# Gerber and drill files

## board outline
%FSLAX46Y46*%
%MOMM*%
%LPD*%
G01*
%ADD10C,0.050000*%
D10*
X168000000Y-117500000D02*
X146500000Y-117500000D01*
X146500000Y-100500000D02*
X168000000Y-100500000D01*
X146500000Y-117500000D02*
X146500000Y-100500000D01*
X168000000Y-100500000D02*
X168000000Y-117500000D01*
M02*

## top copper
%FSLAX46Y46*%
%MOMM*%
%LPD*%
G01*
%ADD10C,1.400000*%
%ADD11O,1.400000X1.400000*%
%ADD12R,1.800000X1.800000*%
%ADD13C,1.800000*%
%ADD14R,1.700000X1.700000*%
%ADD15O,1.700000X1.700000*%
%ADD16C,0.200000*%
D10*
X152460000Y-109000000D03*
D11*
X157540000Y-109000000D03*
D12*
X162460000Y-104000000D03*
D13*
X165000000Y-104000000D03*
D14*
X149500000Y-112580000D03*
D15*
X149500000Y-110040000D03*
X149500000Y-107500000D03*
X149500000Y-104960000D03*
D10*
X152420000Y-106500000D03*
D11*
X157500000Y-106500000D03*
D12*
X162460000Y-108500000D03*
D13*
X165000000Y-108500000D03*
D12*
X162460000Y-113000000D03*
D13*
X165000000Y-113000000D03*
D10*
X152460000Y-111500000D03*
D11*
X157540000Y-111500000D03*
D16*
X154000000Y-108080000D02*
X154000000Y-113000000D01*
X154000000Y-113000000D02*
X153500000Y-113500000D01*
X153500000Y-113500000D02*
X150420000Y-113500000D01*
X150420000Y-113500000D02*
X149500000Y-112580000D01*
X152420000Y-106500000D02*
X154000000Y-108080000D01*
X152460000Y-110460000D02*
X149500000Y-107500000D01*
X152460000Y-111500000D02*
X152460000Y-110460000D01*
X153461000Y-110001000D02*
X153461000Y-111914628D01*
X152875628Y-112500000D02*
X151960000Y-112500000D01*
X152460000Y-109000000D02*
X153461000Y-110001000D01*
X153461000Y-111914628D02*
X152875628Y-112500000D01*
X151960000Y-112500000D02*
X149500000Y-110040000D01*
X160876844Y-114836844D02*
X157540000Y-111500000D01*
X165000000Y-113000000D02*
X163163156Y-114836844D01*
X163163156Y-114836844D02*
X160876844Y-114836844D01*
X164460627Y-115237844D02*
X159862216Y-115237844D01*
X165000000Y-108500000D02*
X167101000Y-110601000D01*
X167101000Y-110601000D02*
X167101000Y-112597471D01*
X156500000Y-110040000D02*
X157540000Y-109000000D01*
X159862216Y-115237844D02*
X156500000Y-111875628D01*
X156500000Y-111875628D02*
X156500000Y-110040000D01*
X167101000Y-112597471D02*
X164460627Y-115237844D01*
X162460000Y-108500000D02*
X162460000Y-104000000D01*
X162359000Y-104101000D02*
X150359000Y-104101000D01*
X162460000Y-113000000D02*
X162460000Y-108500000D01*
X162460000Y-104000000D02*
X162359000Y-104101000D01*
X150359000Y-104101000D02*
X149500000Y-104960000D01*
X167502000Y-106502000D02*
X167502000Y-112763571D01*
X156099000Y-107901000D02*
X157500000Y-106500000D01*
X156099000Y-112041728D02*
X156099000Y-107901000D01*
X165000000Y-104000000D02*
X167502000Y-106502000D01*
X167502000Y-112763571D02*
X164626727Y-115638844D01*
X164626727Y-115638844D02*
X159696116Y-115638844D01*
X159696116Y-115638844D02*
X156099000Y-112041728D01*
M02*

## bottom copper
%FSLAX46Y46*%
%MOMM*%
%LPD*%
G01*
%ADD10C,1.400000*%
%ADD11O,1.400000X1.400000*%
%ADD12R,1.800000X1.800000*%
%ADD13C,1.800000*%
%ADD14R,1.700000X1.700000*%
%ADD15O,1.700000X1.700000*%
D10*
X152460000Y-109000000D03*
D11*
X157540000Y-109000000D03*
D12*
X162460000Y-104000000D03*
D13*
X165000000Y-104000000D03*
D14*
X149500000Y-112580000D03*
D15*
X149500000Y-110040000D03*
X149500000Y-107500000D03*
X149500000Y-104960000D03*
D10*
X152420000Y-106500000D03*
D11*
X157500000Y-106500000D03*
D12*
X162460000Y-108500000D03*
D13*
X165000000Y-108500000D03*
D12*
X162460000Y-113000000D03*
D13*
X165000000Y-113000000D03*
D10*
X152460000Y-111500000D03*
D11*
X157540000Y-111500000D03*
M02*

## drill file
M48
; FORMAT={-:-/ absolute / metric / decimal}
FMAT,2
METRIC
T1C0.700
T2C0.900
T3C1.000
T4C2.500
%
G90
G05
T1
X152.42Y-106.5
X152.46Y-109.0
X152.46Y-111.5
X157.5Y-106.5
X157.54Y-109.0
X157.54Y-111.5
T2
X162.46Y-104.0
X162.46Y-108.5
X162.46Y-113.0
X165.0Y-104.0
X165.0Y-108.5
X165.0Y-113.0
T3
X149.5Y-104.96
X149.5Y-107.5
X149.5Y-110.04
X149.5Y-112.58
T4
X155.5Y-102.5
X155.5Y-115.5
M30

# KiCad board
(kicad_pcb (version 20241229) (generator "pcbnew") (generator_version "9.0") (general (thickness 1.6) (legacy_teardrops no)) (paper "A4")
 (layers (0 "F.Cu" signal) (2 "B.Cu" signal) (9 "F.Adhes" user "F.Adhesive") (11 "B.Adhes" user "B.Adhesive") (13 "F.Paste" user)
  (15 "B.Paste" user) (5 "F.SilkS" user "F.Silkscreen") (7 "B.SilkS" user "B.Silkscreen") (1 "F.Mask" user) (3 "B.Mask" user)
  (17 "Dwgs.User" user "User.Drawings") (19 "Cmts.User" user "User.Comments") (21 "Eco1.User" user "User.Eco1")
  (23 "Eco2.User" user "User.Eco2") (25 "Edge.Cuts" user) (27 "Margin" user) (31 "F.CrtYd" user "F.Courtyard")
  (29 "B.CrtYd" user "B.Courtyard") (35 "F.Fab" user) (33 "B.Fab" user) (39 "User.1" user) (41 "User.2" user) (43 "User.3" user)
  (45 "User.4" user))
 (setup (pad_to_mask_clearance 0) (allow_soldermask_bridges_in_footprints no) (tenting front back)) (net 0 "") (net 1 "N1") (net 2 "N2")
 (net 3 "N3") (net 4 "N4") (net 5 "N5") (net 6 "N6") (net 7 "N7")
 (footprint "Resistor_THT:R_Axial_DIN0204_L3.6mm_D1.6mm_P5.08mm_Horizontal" (layer "F.Cu") (at 152.46 109)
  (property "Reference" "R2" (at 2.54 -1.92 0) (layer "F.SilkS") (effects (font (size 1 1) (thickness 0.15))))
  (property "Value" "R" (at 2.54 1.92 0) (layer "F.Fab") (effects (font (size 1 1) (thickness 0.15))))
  (pad "1" thru_hole circle (at 0 0) (size 1.4 1.4) (drill 0.7) (layers "*.Cu" "*.Mask") (remove_unused_layers no) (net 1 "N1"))
  (pad "2" thru_hole oval (at 5.08 0) (size 1.4 1.4) (drill 0.7) (layers "*.Cu" "*.Mask") (remove_unused_layers no) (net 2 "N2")))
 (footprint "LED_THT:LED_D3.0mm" (layer "F.Cu") (at 162.46 104)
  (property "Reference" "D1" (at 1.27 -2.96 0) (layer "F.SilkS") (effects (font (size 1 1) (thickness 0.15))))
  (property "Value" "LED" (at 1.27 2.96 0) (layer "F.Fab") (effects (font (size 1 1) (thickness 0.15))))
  (pad "1" thru_hole rect (at 0 0) (size 1.8 1.8) (drill 0.9) (layers "*.Cu" "*.Mask") (remove_unused_layers no) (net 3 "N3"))
  (pad "2" thru_hole circle (at 2.54 0) (size 1.8 1.8) (drill 0.9) (layers "*.Cu" "*.Mask") (remove_unused_layers no) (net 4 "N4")))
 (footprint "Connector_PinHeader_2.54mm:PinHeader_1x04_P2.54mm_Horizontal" (layer "F.Cu") (at 149.5 112.58 180)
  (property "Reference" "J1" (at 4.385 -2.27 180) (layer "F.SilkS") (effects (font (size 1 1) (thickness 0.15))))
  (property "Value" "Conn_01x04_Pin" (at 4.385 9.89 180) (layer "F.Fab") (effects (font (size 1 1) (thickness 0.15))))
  (pad "1" thru_hole rect (at 0 0 180) (size 1.7 1.7) (drill 1) (layers "*.Cu" "*.Mask") (remove_unused_layers no) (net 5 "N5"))
  (pad "2" thru_hole oval (at 0 2.54 180) (size 1.7 1.7) (drill 1) (layers "*.Cu" "*.Mask") (remove_unused_layers no) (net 1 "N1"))
  (pad "3" thru_hole oval (at 0 5.08 180) (size 1.7 1.7) (drill 1) (layers "*.Cu" "*.Mask") (remove_unused_layers no) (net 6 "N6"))
  (pad "4" thru_hole oval (at 0 7.62 180) (size 1.7 1.7) (drill 1) (layers "*.Cu" "*.Mask") (remove_unused_layers no) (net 3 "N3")))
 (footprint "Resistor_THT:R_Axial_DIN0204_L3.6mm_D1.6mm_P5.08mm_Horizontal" (layer "F.Cu") (at 152.42 106.5)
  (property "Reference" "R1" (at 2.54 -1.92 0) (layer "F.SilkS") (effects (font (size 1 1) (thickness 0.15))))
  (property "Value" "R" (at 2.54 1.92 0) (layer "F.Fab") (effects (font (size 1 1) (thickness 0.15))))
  (pad "1" thru_hole circle (at 0 0) (size 1.4 1.4) (drill 0.7) (layers "*.Cu" "*.Mask") (remove_unused_layers no) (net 5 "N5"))
  (pad "2" thru_hole oval (at 5.08 0) (size 1.4 1.4) (drill 0.7) (layers "*.Cu" "*.Mask") (remove_unused_layers no) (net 4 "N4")))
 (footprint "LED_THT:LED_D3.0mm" (layer "F.Cu") (at 162.46 108.5)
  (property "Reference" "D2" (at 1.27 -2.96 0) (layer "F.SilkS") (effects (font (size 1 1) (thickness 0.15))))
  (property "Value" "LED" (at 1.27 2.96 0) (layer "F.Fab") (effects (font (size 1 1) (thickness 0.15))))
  (pad "1" thru_hole rect (at 0 0) (size 1.8 1.8) (drill 0.9) (layers "*.Cu" "*.Mask") (remove_unused_layers no) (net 3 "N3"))
  (pad "2" thru_hole circle (at 2.54 0) (size 1.8 1.8) (drill 0.9) (layers "*.Cu" "*.Mask") (remove_unused_layers no) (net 2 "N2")))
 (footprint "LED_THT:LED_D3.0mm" (layer "F.Cu") (at 162.46 113)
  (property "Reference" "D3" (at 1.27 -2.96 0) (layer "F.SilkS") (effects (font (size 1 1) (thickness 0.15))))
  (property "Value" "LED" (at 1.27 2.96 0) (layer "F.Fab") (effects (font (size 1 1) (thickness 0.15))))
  (pad "1" thru_hole rect (at 0 0) (size 1.8 1.8) (drill 0.9) (layers "*.Cu" "*.Mask") (remove_unused_layers no) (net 3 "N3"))
  (pad "2" thru_hole circle (at 2.54 0) (size 1.8 1.8) (drill 0.9) (layers "*.Cu" "*.Mask") (remove_unused_layers no) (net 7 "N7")))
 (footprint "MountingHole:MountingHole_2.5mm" (layer "F.Cu") (at 155.5 102.5)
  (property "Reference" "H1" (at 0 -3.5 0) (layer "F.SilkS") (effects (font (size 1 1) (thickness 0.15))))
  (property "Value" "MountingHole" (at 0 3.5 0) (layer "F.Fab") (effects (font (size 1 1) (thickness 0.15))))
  (pad "" np_thru_hole circle (at 0 0) (size 2.5 2.5) (drill 2.5) (layers "*.Cu" "*.Mask")))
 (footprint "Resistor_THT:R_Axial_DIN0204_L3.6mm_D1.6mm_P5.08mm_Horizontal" (layer "F.Cu") (at 152.46 111.5)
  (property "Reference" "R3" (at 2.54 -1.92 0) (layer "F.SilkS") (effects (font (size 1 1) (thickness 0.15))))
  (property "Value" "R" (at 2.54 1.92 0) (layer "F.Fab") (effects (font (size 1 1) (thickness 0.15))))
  (pad "1" thru_hole circle (at 0 0) (size 1.4 1.4) (drill 0.7) (layers "*.Cu" "*.Mask") (remove_unused_layers no) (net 6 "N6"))
  (pad "2" thru_hole oval (at 5.08 0) (size 1.4 1.4) (drill 0.7) (layers "*.Cu" "*.Mask") (remove_unused_layers no) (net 7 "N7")))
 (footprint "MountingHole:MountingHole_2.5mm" (layer "F.Cu") (at 155.5 115.5)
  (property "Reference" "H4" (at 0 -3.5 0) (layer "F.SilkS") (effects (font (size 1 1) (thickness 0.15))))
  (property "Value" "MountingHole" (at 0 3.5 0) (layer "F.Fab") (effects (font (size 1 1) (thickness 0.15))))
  (pad "" np_thru_hole circle (at 0 0) (size 2.5 2.5) (drill 2.5) (layers "*.Cu" "*.Mask")))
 (gr_line (start 168 117.5) (end 146.5 117.5) (stroke (width 0.05) (type default)) (layer "Edge.Cuts"))
 (gr_line (start 146.5 100.5) (end 168 100.5) (stroke (width 0.05) (type default)) (layer "Edge.Cuts"))
 (gr_line (start 146.5 117.5) (end 146.5 100.5) (stroke (width 0.05) (type default)) (layer "Edge.Cuts"))
 (gr_line (start 168 100.5) (end 168 117.5) (stroke (width 0.05) (type default)) (layer "Edge.Cuts"))
 (segment (start 154 108.08) (end 154 113) (width 0.2) (layer "F.Cu") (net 5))
 (segment (start 154 113) (end 153.5 113.5) (width 0.2) (layer "F.Cu") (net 5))
 (segment (start 153.5 113.5) (end 150.42 113.5) (width 0.2) (layer "F.Cu") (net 5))
 (segment (start 150.42 113.5) (end 149.5 112.58) (width 0.2) (layer "F.Cu") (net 5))
 (segment (start 152.42 106.5) (end 154 108.08) (width 0.2) (layer "F.Cu") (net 5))
 (segment (start 152.46 110.46) (end 149.5 107.5) (width 0.2) (layer "F.Cu") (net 6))
 (segment (start 152.46 111.5) (end 152.46 110.46) (width 0.2) (layer "F.Cu") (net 6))
 (segment (start 153.461 110.001) (end 153.461 111.914628) (width 0.2) (layer "F.Cu") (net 1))
 (segment (start 152.875628 112.5) (end 151.96 112.5) (width 0.2) (layer "F.Cu") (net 1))
 (segment (start 152.46 109) (end 153.461 110.001) (width 0.2) (layer "F.Cu") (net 1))
 (segment (start 153.461 111.914628) (end 152.875628 112.5) (width 0.2) (layer "F.Cu") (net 1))
 (segment (start 151.96 112.5) (end 149.5 110.04) (width 0.2) (layer "F.Cu") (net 1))
 (segment (start 160.876844 114.836844) (end 157.54 111.5) (width 0.2) (layer "F.Cu") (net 7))
 (segment (start 165 113) (end 163.163156 114.836844) (width 0.2) (layer "F.Cu") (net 7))
 (segment (start 163.163156 114.836844) (end 160.876844 114.836844) (width 0.2) (layer "F.Cu") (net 7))
 (segment (start 164.460627 115.237844) (end 159.862216 115.237844) (width 0.2) (layer "F.Cu") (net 2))
 (segment (start 165 108.5) (end 167.101 110.601) (width 0.2) (layer "F.Cu") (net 2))
 (segment (start 167.101 110.601) (end 167.101 112.597471) (width 0.2) (layer "F.Cu") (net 2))
 (segment (start 156.5 110.04) (end 157.54 109) (width 0.2) (layer "F.Cu") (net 2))
 (segment (start 159.862216 115.237844) (end 156.5 111.875628) (width 0.2) (layer "F.Cu") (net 2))
 (segment (start 156.5 111.875628) (end 156.5 110.04) (width 0.2) (layer "F.Cu") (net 2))
 (segment (start 167.101 112.597471) (end 164.460627 115.237844) (width 0.2) (layer "F.Cu") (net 2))
 (segment (start 162.46 108.5) (end 162.46 104) (width 0.2) (layer "F.Cu") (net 3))
 (segment (start 162.359 104.101) (end 150.359 104.101) (width 0.2) (layer "F.Cu") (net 3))
 (segment (start 162.46 113) (end 162.46 108.5) (width 0.2) (layer "F.Cu") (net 3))
 (segment (start 162.46 104) (end 162.359 104.101) (width 0.2) (layer "F.Cu") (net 3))
 (segment (start 150.359 104.101) (end 149.5 104.96) (width 0.2) (layer "F.Cu") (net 3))
 (segment (start 167.502 106.502) (end 167.502 112.763571) (width 0.2) (layer "F.Cu") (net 4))
 (segment (start 156.099 107.901) (end 157.5 106.5) (width 0.2) (layer "F.Cu") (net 4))
 (segment (start 156.099 112.041728) (end 156.099 107.901) (width 0.2) (layer "F.Cu") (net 4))
 (segment (start 165 104) (end 167.502 106.502) (width 0.2) (layer "F.Cu") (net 4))
 (segment (start 167.502 112.763571) (end 164.626727 115.638844) (width 0.2) (layer "F.Cu") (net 4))
 (segment (start 164.626727 115.638844) (end 159.696116 115.638844) (width 0.2) (layer "F.Cu") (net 4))
 (segment (start 159.696116 115.638844) (end 156.099 112.041728) (width 0.2) (layer "F.Cu") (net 4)))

